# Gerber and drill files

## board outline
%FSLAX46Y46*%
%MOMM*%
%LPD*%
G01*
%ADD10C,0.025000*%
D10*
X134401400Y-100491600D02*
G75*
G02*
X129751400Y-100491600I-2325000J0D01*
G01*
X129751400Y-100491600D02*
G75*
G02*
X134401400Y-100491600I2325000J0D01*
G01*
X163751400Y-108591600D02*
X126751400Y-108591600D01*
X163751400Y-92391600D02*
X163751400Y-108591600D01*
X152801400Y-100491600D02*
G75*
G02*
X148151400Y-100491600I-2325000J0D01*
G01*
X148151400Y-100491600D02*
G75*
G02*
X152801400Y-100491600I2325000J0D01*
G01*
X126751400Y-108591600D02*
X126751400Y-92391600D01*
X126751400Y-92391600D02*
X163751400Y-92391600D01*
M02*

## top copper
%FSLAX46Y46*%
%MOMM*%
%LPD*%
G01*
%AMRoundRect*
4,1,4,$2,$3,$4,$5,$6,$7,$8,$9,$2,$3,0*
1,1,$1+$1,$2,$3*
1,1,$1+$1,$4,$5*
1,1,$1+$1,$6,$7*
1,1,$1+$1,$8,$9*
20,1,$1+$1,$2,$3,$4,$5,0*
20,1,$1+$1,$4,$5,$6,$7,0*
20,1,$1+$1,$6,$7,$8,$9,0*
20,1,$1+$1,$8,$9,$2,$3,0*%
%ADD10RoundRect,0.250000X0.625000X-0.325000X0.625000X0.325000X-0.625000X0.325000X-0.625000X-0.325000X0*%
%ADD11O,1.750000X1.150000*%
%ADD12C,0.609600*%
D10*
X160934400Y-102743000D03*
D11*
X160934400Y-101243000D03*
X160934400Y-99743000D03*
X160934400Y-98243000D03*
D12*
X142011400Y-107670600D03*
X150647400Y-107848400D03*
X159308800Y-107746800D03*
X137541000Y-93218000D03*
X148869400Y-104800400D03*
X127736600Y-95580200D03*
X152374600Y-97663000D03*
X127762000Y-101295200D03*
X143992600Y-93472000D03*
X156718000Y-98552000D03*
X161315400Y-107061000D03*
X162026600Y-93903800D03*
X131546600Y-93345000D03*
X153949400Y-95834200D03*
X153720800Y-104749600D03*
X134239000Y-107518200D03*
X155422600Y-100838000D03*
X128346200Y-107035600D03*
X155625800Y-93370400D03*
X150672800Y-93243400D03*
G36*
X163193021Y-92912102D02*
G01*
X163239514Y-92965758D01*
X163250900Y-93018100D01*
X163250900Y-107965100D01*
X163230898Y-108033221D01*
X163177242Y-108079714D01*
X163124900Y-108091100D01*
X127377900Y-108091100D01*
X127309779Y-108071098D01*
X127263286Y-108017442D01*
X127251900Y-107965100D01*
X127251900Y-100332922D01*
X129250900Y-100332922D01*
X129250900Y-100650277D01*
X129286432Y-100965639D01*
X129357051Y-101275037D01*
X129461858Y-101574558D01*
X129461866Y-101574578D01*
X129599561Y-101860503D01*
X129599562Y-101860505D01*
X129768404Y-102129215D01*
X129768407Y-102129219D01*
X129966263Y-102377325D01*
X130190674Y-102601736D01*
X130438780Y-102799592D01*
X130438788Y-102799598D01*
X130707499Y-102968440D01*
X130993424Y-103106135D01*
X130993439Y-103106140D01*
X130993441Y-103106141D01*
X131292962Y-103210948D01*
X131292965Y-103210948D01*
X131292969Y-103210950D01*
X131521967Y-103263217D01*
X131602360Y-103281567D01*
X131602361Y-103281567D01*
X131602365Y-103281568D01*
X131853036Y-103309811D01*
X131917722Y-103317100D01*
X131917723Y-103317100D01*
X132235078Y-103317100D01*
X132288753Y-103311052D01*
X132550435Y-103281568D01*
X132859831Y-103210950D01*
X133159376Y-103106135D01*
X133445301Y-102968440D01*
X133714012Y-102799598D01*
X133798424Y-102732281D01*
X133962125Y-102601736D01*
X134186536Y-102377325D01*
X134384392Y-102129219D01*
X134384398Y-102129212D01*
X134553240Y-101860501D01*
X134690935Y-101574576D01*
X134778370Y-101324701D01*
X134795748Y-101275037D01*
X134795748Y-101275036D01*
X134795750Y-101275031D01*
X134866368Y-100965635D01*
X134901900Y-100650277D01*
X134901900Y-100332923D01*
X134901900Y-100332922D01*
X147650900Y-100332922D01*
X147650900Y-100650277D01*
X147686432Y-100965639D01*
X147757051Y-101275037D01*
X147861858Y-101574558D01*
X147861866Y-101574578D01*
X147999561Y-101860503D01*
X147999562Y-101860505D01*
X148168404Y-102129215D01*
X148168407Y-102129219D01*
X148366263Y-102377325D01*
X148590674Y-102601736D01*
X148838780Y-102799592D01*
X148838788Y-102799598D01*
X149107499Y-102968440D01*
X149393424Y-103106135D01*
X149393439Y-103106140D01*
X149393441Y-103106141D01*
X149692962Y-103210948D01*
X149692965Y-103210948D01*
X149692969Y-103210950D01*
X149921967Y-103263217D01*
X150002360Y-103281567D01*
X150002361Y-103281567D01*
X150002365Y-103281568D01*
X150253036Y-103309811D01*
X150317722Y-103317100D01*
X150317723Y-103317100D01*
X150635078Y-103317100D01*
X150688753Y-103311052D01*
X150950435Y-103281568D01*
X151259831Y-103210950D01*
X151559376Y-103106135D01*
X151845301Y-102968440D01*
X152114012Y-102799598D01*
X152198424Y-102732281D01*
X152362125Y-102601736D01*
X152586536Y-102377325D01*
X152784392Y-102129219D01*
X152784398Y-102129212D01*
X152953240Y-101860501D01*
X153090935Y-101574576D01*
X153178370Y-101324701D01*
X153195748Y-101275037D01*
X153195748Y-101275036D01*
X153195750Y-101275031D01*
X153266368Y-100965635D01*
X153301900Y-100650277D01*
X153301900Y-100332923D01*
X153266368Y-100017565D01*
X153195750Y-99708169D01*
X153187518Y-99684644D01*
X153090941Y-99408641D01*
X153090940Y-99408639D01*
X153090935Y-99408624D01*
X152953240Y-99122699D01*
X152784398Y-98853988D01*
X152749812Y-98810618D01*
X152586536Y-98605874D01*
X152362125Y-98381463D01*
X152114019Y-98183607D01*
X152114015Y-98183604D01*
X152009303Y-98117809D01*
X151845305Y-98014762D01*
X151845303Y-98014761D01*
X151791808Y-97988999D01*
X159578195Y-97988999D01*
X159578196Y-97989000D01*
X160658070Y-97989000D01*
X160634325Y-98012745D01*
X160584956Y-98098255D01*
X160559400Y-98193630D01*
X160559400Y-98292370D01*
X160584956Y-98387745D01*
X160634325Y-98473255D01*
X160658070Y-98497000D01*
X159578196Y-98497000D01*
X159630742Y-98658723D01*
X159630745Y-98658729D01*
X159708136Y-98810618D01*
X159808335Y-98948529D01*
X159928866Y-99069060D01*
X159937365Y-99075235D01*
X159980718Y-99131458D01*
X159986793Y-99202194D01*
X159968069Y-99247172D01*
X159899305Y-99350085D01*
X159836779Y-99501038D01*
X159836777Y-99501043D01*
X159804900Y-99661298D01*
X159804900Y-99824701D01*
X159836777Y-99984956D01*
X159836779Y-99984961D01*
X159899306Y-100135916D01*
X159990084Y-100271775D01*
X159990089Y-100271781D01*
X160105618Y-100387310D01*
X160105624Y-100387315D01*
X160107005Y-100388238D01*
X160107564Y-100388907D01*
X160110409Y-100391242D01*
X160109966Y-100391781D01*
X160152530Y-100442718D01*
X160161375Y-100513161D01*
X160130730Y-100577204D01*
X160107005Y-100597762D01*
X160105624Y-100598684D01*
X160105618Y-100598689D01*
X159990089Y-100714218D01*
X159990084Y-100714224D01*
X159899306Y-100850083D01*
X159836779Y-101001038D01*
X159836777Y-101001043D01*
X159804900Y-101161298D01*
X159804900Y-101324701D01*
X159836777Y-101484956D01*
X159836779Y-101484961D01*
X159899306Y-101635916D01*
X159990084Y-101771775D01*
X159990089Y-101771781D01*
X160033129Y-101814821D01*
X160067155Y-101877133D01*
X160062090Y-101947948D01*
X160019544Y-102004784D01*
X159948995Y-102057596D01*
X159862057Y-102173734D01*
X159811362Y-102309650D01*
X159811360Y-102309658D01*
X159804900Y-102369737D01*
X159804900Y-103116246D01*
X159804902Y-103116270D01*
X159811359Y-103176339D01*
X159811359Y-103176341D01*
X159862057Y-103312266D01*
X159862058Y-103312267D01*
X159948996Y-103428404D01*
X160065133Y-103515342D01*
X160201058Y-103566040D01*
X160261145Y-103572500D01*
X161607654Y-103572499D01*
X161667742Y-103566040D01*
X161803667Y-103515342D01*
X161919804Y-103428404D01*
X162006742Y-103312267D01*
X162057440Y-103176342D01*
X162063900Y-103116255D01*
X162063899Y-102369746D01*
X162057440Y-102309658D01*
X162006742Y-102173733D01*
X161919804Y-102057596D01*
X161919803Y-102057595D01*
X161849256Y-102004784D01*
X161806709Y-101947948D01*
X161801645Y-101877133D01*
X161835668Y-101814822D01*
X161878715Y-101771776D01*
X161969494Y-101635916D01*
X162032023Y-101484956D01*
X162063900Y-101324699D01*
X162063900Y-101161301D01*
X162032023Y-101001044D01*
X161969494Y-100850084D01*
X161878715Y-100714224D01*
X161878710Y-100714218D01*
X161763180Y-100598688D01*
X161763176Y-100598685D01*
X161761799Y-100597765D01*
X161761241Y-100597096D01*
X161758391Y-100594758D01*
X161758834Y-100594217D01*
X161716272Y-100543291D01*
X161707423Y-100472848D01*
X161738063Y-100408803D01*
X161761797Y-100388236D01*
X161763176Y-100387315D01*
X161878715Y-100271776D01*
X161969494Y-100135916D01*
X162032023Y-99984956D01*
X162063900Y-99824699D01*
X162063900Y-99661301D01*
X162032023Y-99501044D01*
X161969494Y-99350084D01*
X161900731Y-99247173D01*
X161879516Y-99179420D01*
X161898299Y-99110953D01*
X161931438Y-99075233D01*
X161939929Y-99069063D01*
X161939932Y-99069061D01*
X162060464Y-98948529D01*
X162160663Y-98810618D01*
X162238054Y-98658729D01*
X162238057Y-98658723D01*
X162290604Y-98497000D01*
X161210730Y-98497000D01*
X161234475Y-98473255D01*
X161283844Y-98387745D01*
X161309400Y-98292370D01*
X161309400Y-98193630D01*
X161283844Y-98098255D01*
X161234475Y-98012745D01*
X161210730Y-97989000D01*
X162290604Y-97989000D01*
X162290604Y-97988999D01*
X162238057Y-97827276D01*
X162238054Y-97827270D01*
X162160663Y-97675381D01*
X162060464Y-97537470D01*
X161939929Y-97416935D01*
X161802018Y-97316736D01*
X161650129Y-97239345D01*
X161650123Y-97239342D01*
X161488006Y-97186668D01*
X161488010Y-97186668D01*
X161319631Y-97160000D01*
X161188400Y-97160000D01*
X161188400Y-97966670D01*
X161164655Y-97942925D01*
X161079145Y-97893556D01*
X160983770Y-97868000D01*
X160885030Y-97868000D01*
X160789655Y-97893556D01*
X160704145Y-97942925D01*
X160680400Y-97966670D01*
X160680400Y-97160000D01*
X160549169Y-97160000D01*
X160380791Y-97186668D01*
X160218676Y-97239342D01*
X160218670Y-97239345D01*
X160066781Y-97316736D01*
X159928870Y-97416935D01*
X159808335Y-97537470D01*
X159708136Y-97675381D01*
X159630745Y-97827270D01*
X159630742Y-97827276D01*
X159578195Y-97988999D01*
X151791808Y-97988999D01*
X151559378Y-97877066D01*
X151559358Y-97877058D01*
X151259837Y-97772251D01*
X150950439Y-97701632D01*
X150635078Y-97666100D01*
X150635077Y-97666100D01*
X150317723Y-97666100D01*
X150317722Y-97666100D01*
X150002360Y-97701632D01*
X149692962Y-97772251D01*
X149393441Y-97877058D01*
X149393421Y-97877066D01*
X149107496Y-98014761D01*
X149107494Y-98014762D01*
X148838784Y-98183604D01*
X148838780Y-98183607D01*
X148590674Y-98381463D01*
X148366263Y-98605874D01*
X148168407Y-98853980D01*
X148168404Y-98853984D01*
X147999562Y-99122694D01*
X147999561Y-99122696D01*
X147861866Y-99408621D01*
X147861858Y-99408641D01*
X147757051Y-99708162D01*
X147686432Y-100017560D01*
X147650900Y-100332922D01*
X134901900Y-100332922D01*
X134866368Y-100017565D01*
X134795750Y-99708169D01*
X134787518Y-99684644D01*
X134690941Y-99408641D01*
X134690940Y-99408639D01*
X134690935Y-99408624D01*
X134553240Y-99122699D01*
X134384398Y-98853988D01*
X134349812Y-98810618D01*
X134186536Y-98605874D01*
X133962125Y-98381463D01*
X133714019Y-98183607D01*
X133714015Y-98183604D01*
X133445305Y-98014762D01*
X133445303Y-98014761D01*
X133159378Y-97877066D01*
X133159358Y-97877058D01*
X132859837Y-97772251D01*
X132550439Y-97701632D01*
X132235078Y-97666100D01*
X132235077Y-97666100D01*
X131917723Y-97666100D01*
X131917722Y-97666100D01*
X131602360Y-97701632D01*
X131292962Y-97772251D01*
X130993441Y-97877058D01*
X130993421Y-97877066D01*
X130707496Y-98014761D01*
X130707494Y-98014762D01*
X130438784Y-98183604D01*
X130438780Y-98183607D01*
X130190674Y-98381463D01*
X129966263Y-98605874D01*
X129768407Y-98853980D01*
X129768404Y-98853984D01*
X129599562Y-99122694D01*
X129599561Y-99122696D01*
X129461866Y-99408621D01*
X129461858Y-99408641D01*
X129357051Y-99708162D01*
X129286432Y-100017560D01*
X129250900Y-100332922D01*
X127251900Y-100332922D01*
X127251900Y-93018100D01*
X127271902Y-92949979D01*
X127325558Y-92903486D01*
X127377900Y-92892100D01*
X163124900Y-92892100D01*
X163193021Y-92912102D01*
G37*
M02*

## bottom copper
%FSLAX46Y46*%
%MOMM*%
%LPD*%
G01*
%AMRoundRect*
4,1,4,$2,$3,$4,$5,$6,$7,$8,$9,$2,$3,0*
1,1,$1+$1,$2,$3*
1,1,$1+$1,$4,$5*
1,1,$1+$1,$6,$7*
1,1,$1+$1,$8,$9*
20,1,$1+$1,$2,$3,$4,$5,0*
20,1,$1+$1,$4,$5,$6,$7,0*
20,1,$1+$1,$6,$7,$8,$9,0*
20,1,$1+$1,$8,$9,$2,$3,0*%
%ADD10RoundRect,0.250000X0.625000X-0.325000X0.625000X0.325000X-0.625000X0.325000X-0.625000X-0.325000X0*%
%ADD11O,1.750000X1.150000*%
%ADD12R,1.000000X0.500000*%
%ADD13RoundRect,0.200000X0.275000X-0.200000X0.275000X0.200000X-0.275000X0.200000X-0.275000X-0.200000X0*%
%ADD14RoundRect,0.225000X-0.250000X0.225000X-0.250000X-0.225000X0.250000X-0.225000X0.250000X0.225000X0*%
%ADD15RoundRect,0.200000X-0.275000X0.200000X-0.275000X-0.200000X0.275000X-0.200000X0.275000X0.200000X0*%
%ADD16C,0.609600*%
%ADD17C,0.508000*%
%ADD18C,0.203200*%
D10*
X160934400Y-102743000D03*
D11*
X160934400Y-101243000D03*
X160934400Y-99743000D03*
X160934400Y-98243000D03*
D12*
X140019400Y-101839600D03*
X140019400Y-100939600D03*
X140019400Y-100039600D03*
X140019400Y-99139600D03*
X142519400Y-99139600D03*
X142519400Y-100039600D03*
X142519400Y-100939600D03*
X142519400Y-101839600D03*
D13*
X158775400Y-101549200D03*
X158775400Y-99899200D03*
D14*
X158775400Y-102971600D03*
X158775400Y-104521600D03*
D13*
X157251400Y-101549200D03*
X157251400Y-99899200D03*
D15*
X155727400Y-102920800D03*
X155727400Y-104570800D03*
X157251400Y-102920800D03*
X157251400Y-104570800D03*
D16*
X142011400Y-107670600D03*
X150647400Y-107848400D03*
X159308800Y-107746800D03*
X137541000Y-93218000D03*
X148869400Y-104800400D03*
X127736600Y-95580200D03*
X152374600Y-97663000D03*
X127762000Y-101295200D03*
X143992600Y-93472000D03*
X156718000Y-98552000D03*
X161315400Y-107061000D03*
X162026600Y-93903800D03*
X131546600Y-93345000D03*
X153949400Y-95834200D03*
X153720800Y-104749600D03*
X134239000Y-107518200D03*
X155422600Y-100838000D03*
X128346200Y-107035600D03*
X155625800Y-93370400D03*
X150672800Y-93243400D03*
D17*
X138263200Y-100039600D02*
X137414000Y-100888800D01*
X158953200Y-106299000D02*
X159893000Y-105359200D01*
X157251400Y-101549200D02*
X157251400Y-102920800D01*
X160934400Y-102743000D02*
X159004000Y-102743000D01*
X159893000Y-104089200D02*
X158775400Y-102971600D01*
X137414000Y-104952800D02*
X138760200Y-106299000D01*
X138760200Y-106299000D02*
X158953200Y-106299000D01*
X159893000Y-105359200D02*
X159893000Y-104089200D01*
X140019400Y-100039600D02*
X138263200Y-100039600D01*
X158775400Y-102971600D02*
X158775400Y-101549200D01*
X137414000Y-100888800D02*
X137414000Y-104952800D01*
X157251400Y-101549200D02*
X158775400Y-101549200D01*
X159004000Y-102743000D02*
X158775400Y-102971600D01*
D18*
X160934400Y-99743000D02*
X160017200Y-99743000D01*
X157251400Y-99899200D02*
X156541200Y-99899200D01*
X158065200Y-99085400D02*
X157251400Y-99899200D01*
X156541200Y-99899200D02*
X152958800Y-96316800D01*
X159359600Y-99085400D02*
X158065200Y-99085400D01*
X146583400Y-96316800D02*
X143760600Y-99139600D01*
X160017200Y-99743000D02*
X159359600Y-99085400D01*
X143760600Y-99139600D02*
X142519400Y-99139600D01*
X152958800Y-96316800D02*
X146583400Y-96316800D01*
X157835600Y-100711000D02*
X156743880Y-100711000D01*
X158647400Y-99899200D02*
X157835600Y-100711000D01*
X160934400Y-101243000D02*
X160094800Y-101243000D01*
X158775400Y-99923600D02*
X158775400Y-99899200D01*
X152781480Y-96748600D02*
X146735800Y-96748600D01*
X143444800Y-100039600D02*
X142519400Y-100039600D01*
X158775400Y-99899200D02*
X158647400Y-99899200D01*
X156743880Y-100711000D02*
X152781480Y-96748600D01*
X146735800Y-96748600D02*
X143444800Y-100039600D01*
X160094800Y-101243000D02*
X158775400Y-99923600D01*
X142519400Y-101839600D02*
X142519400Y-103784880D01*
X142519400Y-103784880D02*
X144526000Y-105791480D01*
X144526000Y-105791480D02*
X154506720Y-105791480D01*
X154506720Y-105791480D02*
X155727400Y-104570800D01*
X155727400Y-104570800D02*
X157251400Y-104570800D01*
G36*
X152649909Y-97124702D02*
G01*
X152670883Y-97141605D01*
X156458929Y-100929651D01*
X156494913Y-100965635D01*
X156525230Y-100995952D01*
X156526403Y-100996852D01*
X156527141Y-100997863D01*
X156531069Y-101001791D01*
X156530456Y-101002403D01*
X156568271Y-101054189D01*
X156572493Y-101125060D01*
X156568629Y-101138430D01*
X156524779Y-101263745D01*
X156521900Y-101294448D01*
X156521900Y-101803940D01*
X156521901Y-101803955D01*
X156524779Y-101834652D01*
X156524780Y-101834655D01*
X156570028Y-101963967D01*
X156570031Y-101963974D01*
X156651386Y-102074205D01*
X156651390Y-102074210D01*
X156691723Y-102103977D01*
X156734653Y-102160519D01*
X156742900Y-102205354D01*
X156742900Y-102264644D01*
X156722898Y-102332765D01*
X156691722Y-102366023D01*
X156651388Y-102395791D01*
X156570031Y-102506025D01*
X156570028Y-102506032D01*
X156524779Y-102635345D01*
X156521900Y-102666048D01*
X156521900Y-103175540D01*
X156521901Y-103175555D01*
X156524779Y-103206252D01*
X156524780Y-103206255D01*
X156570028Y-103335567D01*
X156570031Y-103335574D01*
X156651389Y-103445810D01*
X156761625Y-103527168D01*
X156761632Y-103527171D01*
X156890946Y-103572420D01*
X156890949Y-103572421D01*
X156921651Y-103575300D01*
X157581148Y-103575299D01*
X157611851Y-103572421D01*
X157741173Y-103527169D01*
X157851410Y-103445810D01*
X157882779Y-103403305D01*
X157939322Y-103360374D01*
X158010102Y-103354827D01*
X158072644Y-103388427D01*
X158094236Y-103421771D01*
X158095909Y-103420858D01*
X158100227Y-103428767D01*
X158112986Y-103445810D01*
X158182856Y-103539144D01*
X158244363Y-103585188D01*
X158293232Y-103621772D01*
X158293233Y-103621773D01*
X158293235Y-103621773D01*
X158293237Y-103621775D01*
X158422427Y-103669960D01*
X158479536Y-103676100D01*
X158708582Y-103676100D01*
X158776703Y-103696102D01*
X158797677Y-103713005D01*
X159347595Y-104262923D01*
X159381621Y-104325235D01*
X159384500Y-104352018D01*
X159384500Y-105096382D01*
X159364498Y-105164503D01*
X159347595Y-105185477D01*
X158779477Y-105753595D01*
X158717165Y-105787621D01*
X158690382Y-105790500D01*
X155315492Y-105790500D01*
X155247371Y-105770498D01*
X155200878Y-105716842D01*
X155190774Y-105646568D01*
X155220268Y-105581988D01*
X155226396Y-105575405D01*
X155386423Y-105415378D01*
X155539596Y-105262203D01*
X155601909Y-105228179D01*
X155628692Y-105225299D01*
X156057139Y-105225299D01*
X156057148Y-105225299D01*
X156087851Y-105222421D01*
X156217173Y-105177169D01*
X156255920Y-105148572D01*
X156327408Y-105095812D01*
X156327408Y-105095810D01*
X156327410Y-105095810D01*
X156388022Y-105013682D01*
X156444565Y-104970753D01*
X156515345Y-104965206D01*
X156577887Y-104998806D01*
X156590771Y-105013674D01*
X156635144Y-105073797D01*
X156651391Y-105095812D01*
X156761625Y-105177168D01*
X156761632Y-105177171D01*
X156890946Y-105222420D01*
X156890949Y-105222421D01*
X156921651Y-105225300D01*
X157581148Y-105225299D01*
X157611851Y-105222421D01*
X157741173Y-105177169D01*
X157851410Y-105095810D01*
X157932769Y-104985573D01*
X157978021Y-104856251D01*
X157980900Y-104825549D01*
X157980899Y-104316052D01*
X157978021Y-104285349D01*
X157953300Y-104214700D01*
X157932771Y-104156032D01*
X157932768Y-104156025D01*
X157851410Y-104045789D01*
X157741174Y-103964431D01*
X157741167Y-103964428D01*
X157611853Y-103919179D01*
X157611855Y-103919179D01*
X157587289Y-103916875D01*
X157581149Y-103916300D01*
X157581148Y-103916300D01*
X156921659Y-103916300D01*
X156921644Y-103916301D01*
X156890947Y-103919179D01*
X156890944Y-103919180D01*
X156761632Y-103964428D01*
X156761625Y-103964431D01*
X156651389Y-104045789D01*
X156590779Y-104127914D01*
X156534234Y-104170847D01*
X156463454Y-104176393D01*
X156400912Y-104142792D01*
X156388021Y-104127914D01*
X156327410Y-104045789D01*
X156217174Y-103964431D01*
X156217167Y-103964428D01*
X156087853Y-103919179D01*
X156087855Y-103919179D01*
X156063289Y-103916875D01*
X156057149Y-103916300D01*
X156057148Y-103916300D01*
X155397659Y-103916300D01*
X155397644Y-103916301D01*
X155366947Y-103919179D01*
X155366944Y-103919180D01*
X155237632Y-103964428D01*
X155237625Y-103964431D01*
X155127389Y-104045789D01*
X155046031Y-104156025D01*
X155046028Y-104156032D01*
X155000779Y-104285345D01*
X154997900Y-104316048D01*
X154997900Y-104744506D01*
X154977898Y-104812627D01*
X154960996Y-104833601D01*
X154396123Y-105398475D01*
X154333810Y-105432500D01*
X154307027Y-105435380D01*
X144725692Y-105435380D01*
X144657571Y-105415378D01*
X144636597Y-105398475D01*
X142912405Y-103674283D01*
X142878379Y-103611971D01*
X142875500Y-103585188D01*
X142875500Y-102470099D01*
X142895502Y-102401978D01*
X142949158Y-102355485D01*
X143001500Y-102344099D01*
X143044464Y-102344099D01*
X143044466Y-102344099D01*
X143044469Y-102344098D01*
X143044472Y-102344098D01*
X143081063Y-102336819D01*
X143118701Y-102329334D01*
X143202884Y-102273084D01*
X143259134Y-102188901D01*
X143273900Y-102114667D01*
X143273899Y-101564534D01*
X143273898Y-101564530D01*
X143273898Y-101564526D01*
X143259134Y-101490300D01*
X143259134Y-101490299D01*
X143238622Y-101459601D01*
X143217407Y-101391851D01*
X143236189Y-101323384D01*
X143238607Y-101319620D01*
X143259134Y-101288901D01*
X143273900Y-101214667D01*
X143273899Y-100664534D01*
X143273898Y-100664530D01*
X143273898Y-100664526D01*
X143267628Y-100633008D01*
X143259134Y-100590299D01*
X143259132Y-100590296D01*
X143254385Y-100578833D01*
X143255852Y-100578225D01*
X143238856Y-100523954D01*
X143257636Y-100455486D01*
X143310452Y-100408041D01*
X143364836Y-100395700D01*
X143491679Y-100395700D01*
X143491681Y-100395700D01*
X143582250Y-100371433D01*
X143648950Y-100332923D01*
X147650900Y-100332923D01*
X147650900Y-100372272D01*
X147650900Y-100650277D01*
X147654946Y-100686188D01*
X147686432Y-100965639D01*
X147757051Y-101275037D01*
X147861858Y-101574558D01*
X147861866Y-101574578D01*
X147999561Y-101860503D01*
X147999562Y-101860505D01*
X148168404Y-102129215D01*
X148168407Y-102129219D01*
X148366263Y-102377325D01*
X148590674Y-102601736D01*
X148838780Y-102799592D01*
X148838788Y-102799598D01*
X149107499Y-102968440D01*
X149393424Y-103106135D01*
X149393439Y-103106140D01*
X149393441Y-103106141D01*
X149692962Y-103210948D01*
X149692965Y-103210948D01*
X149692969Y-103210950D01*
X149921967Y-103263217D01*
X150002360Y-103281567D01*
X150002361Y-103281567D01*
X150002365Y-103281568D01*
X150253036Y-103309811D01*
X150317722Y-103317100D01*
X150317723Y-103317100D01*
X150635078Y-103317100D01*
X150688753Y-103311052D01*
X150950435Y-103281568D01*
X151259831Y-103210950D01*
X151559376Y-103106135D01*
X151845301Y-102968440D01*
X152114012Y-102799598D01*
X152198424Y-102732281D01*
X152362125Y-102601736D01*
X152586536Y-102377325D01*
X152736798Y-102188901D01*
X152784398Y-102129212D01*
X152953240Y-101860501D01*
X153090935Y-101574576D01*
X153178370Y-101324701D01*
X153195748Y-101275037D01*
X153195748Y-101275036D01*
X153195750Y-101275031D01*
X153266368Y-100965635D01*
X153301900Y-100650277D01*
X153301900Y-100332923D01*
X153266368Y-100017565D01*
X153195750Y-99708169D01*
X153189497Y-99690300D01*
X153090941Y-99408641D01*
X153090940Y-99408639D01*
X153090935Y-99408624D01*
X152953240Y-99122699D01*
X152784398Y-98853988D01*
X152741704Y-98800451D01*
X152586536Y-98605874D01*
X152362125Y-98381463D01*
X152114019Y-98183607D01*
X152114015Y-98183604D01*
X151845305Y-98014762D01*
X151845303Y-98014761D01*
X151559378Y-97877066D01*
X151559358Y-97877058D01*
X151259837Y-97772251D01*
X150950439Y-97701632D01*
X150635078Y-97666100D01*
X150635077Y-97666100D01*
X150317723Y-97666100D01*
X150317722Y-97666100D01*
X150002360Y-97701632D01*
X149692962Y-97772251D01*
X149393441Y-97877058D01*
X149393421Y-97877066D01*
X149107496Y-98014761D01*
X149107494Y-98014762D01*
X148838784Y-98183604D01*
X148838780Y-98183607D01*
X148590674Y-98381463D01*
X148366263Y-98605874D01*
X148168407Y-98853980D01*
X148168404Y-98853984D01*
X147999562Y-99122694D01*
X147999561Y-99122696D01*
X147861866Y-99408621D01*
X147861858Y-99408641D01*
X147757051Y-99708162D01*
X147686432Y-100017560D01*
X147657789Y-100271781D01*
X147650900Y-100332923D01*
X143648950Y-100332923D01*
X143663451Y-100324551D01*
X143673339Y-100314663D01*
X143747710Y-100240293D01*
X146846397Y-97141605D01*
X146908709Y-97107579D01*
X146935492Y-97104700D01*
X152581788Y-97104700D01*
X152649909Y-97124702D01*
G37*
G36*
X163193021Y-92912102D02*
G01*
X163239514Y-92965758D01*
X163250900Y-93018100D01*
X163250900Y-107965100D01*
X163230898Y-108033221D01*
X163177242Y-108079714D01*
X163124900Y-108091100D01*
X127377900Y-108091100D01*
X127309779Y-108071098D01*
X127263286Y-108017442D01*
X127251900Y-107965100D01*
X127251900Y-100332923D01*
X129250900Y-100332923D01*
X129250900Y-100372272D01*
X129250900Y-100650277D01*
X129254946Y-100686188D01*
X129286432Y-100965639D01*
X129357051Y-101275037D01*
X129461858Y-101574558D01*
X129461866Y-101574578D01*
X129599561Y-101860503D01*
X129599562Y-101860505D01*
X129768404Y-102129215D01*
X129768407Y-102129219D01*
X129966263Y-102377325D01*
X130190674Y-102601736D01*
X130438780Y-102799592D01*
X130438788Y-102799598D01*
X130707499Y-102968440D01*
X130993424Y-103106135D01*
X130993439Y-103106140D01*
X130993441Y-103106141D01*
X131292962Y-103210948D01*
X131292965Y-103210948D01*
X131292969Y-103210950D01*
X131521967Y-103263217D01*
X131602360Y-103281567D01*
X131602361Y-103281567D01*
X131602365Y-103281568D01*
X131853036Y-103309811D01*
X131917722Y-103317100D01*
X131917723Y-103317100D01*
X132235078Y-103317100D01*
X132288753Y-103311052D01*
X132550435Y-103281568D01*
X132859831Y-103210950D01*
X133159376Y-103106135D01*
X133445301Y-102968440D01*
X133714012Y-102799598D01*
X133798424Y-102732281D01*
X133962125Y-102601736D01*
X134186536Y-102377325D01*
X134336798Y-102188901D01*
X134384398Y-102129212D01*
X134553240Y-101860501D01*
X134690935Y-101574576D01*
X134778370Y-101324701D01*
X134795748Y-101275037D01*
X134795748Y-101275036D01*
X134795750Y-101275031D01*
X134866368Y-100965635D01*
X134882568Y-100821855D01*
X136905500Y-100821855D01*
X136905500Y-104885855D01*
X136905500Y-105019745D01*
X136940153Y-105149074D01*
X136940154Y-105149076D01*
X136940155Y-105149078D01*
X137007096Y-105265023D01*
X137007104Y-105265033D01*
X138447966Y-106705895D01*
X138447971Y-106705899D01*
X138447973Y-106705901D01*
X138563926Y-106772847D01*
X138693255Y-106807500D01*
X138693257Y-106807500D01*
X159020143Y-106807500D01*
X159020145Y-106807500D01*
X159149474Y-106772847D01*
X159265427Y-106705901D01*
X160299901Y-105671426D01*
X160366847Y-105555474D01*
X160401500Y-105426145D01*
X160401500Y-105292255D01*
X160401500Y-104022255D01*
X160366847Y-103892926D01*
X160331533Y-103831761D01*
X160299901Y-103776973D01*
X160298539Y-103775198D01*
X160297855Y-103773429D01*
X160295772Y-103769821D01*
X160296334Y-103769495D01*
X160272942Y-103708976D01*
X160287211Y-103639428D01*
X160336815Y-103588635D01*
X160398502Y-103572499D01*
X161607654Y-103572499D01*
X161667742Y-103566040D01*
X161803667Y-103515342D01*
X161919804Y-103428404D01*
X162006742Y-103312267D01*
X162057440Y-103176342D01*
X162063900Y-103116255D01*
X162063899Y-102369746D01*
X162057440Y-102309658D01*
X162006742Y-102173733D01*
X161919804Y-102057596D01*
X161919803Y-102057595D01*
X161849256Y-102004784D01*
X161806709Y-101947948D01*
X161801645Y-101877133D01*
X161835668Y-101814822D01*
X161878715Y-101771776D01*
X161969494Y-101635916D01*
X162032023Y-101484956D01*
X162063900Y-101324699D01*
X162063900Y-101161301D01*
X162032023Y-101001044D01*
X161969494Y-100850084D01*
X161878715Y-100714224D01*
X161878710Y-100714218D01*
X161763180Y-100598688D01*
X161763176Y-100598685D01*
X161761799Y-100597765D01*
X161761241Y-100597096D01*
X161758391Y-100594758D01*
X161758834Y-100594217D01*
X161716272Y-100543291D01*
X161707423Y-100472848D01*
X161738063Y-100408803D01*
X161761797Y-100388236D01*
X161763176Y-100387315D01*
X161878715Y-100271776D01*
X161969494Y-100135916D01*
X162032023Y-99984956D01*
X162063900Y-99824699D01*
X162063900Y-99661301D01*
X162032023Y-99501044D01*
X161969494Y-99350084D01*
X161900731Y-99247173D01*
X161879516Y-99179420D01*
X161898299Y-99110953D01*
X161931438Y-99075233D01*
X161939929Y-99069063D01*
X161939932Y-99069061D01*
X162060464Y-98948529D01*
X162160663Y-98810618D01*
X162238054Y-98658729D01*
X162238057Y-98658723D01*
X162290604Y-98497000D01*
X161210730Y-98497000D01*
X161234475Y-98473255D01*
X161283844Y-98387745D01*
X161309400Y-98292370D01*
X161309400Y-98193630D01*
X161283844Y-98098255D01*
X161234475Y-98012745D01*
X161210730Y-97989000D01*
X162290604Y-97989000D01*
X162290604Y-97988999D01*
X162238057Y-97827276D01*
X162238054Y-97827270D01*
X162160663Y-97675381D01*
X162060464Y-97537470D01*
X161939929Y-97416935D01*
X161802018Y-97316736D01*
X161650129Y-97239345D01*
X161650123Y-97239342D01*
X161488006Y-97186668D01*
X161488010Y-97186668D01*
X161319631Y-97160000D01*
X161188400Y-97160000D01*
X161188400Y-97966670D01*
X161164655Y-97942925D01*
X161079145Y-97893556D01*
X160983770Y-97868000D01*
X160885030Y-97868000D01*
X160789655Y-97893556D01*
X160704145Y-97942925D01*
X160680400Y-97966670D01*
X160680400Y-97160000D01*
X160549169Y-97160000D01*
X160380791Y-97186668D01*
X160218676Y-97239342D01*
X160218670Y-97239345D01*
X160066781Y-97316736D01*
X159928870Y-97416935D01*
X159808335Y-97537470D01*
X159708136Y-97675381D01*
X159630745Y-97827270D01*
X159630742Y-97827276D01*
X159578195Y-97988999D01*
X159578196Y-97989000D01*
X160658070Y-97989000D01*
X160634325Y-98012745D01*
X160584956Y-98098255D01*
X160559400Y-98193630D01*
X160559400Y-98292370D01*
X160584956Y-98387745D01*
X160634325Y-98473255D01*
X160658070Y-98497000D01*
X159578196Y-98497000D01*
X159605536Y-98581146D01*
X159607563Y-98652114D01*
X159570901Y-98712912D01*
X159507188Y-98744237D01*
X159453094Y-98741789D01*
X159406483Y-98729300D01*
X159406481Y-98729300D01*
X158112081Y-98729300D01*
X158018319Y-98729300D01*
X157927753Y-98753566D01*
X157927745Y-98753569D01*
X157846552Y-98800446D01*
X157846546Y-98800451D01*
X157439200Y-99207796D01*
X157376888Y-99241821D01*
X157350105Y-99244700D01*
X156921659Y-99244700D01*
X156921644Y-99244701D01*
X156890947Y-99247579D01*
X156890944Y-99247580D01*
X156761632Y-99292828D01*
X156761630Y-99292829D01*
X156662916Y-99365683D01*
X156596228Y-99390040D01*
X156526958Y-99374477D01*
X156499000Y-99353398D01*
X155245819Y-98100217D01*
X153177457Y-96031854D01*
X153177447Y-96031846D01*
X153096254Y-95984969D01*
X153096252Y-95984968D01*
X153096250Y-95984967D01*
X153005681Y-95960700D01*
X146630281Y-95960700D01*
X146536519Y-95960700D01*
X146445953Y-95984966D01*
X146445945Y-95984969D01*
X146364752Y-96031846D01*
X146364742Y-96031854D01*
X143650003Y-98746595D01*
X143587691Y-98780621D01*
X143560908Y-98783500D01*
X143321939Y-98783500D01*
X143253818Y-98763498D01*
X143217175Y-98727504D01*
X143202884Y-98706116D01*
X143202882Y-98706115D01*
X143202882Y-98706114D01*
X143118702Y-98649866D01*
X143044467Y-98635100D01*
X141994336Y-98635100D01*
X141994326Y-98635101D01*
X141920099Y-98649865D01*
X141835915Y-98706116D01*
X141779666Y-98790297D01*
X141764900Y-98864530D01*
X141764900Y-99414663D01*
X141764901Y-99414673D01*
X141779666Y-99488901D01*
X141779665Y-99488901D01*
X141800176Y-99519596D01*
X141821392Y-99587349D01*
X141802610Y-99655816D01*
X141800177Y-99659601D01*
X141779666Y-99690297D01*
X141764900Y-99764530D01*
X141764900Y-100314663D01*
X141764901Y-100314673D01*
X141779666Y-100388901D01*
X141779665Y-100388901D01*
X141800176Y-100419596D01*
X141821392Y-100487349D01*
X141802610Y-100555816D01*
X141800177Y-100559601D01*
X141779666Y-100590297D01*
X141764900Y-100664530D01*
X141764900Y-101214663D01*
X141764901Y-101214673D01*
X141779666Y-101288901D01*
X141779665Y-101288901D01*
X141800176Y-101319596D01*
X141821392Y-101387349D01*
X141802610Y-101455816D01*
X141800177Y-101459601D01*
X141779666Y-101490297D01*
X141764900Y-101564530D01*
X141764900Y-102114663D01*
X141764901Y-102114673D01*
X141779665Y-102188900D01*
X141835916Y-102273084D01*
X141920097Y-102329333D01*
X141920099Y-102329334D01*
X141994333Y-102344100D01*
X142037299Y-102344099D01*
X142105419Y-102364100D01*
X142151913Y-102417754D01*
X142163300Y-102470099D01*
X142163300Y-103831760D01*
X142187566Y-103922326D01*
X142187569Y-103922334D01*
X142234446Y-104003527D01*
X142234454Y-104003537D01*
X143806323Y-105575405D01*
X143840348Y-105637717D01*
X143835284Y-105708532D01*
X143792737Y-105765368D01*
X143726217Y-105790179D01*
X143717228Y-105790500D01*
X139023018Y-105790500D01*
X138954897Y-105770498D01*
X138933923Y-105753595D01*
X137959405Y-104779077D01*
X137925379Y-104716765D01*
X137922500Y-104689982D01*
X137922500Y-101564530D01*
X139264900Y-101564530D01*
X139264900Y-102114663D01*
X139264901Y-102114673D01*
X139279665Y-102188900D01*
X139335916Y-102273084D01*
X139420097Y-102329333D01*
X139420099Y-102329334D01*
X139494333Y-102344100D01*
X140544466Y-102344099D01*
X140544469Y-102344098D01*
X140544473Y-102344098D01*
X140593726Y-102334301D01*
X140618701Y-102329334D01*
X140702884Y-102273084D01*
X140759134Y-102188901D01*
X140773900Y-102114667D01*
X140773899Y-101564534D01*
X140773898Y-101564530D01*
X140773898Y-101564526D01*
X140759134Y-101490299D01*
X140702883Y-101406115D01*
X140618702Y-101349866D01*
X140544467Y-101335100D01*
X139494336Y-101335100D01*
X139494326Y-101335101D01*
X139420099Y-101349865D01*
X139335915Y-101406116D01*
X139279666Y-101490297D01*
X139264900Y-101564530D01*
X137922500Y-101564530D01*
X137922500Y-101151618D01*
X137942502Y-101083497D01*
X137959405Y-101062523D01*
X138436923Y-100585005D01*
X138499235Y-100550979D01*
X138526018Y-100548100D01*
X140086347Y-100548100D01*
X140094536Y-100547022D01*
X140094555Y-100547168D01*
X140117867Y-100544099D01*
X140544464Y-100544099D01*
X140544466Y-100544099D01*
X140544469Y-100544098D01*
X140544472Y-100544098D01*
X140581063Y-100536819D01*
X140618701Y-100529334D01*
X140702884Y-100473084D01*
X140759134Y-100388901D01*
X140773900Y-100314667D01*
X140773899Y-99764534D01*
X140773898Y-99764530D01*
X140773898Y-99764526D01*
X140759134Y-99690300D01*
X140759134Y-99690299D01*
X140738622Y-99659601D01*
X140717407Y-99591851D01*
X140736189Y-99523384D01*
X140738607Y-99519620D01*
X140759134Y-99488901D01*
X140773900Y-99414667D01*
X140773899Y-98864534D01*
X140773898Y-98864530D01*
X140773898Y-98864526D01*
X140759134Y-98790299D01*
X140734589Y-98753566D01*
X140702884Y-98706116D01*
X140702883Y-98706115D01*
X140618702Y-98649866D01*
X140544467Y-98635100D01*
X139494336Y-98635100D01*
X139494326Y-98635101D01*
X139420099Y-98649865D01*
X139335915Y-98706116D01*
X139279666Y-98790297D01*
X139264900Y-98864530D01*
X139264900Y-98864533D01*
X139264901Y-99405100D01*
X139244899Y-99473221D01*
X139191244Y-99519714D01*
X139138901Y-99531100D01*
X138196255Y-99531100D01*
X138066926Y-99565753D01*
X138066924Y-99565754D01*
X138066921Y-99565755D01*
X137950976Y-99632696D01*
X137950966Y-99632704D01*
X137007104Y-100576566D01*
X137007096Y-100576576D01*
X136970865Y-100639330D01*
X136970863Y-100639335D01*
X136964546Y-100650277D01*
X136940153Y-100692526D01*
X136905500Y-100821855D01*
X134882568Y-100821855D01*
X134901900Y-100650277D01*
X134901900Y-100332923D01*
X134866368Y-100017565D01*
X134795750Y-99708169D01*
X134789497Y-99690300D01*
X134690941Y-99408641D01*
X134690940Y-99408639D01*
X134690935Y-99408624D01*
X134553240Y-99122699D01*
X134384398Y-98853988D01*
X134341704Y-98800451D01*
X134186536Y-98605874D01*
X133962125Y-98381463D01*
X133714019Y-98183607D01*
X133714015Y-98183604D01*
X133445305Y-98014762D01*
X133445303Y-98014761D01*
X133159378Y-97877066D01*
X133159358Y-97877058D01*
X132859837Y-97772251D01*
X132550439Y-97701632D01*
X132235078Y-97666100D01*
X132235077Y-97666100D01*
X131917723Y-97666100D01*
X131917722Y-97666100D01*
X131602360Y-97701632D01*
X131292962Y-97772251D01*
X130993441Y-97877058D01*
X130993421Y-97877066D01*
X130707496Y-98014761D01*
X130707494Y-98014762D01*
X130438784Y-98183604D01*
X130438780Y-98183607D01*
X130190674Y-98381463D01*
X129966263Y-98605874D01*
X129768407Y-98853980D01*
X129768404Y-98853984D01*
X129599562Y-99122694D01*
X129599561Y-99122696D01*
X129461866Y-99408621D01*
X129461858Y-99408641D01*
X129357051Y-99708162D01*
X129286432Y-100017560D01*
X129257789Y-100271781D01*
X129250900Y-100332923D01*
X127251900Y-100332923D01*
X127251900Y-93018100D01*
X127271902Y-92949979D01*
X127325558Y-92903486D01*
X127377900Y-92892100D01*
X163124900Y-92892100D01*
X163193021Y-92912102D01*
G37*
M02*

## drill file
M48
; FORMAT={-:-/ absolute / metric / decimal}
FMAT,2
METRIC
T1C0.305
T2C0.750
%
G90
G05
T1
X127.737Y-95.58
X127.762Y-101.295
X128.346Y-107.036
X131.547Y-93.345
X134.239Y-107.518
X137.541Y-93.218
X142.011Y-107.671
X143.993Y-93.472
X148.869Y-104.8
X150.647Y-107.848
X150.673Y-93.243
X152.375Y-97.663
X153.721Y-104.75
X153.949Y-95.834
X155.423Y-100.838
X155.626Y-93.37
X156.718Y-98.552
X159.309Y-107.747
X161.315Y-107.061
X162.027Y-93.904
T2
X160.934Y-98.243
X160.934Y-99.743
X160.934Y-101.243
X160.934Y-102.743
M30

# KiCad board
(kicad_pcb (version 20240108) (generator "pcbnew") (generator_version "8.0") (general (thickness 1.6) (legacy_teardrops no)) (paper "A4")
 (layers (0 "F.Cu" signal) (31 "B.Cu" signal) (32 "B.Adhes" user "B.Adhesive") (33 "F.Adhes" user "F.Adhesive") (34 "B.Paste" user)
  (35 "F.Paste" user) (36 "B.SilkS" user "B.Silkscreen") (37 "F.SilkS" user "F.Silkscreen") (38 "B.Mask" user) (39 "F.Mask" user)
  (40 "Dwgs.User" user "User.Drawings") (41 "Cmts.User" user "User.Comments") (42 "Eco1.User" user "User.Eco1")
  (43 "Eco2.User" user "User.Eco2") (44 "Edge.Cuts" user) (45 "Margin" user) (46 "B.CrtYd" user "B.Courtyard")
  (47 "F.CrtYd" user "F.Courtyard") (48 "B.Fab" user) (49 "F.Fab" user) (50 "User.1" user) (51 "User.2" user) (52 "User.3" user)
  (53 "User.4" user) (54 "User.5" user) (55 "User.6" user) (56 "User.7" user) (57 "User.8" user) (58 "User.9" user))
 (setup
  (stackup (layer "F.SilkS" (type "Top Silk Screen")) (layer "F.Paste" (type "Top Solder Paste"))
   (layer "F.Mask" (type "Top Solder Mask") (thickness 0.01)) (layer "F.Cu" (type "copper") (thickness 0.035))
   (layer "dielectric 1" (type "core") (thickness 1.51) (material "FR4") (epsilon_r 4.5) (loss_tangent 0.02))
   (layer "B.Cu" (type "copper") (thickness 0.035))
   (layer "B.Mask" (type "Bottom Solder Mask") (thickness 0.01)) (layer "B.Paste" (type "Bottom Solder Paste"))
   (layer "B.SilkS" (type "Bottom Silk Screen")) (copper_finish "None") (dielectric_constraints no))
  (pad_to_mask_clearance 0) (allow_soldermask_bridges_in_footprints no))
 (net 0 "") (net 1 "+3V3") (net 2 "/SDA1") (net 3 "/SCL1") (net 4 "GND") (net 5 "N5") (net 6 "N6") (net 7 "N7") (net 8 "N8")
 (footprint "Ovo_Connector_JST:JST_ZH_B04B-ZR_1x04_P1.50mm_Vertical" (layer "F.Cu") (at 160.9344 102.743 90)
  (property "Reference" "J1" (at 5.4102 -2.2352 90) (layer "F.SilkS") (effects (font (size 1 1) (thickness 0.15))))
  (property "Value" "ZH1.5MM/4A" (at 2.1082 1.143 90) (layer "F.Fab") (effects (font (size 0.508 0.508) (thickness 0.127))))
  (pad "1" thru_hole roundrect (at 0 0 90) (size 1.15 1.75) (drill 0.75) (layers "*.Cu" "*.Mask") (remove_unused_layers no)
   (roundrect_rratio 0.2173913043) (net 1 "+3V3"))
  (pad "2" thru_hole oval (at 1.5 0 90) (size 1.15 1.75) (drill 0.75) (layers "*.Cu" "*.Mask") (remove_unused_layers no) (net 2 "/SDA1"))
  (pad "3" thru_hole oval (at 3 0 90) (size 1.15 1.75) (drill 0.75) (layers "*.Cu" "*.Mask") (remove_unused_layers no) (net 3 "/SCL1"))
  (pad "4" thru_hole oval (at 4.5 0 90) (size 1.15 1.75) (drill 0.75) (layers "*.Cu" "*.Mask") (remove_unused_layers no) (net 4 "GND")))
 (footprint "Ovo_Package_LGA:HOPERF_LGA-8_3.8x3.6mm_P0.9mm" (layer "B.Cu") (at 141.2694 100.4896)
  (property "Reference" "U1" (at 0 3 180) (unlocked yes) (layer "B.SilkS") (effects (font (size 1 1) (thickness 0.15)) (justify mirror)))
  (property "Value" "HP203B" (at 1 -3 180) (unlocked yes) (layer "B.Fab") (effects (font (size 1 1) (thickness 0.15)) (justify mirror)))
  (pad "1" smd rect (at -1.25 1.35) (size 1 0.5) (layers "B.Cu" "B.Paste" "B.Mask") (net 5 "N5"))
  (pad "2" smd rect (at -1.25 0.45) (size 1 0.5) (layers "B.Cu" "B.Paste" "B.Mask") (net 4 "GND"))
  (pad "3" smd rect (at -1.25 -0.45) (size 1 0.5) (layers "B.Cu" "B.Paste" "B.Mask") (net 1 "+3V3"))
  (pad "4" smd rect (at -1.25 -1.35) (size 1 0.5) (layers "B.Cu" "B.Paste" "B.Mask") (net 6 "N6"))
  (pad "5" smd rect (at 1.25 -1.35) (size 1 0.5) (layers "B.Cu" "B.Paste" "B.Mask") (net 3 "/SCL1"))
  (pad "6" smd rect (at 1.25 -0.45) (size 1 0.5) (layers "B.Cu" "B.Paste" "B.Mask") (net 2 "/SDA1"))
  (pad "7" smd rect (at 1.25 0.45) (size 1 0.5) (layers "B.Cu" "B.Paste" "B.Mask") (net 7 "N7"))
  (pad "8" smd rect (at 1.25 1.35) (size 1 0.5) (layers "B.Cu" "B.Paste" "B.Mask") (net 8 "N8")))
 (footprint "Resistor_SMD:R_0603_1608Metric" (layer "B.Cu") (at 158.7754 100.7242 90)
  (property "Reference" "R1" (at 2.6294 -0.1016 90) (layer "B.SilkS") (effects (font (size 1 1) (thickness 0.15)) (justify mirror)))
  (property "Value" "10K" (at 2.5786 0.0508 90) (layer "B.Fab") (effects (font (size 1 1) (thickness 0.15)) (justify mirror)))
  (pad "1" smd roundrect (at -0.825 0 90) (size 0.8 0.95) (layers "B.Cu" "B.Paste" "B.Mask") (roundrect_rratio 0.25) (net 1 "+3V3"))
  (pad "2" smd roundrect (at 0.825 0 90) (size 0.8 0.95) (layers "B.Cu" "B.Paste" "B.Mask") (roundrect_rratio 0.25) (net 2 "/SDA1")))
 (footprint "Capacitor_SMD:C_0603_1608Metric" (layer "B.Cu") (at 158.7754 103.7466 -90)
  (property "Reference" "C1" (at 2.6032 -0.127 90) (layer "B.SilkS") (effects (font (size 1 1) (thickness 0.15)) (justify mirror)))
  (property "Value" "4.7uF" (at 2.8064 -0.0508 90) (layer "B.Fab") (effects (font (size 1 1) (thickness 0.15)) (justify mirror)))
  (pad "1" smd roundrect (at -0.775 0 270) (size 0.9 0.95) (layers "B.Cu" "B.Paste" "B.Mask") (roundrect_rratio 0.25) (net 1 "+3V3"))
  (pad "2" smd roundrect (at 0.775 0 270) (size 0.9 0.95) (layers "B.Cu" "B.Paste" "B.Mask") (roundrect_rratio 0.25) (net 4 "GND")))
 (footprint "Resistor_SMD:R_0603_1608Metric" (layer "B.Cu") (at 157.2514 100.7242 90)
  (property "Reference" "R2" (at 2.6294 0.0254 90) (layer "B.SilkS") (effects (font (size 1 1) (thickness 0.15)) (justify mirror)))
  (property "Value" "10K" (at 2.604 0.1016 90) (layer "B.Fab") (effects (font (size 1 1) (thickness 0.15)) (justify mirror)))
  (pad "1" smd roundrect (at -0.825 0 90) (size 0.8 0.95) (layers "B.Cu" "B.Paste" "B.Mask") (roundrect_rratio 0.25) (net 1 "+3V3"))
  (pad "2" smd roundrect (at 0.825 0 90) (size 0.8 0.95) (layers "B.Cu" "B.Paste" "B.Mask") (roundrect_rratio 0.25) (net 3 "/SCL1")))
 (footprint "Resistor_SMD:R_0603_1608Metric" (layer "B.Cu") (at 155.7274 103.7458 -90)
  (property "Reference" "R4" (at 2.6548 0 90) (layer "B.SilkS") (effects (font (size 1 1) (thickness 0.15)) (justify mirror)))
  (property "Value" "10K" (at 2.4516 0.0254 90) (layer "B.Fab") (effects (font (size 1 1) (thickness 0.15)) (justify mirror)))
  (pad "1" smd roundrect (at -0.825 0 270) (size 0.8 0.95) (layers "B.Cu" "B.Paste" "B.Mask") (roundrect_rratio 0.25) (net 4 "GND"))
  (pad "2" smd roundrect (at 0.825 0 270) (size 0.8 0.95) (layers "B.Cu" "B.Paste" "B.Mask") (roundrect_rratio 0.25) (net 8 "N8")))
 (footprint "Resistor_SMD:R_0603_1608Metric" (layer "B.Cu") (at 157.2514 103.7458 -90)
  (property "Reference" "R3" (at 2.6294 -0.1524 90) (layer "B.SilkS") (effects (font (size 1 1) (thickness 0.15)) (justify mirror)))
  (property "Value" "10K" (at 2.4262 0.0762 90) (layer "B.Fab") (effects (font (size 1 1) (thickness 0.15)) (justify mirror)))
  (pad "1" smd roundrect (at -0.825 0 270) (size 0.8 0.95) (layers "B.Cu" "B.Paste" "B.Mask") (roundrect_rratio 0.25) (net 1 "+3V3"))
  (pad "2" smd roundrect (at 0.825 0 270) (size 0.8 0.95) (layers "B.Cu" "B.Paste" "B.Mask") (roundrect_rratio 0.25) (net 8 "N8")))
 (gr_circle (center 132.0764 100.4916) (end 134.4014 100.4916) (stroke (width 0.025) (type solid)) (fill none) (layer "Edge.Cuts"))
 (gr_line (start 163.7514 108.5916) (end 126.7514 108.5916) (stroke (width 0.025) (type solid)) (layer "Edge.Cuts"))
 (gr_line (start 163.7514 92.3916) (end 163.7514 108.5916) (stroke (width 0.025) (type solid)) (layer "Edge.Cuts"))
 (gr_circle (center 150.4764 100.4916) (end 152.8014 100.4916) (stroke (width 0.025) (type solid)) (fill none) (layer "Edge.Cuts"))
 (gr_line (start 126.7514 108.5916) (end 126.7514 92.3916) (stroke (width 0.025) (type solid)) (layer "Edge.Cuts"))
 (gr_line (start 126.7514 92.3916) (end 163.7514 92.3916) (stroke (width 0.025) (type solid)) (layer "Edge.Cuts"))
 (segment (start 138.2632 100.0396) (end 137.414 100.8888) (width 0.508) (layer "B.Cu") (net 1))
 (segment (start 158.9532 106.299) (end 159.893 105.3592) (width 0.508) (layer "B.Cu") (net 1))
 (segment (start 157.2514 101.5492) (end 157.2514 102.9208) (width 0.508) (layer "B.Cu") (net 1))
 (segment (start 160.9344 102.743) (end 159.004 102.743) (width 0.508) (layer "B.Cu") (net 1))
 (segment (start 159.893 104.0892) (end 158.7754 102.9716) (width 0.508) (layer "B.Cu") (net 1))
 (segment (start 137.414 104.9528) (end 138.7602 106.299) (width 0.508) (layer "B.Cu") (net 1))
 (segment (start 138.7602 106.299) (end 158.9532 106.299) (width 0.508) (layer "B.Cu") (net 1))
 (segment (start 159.893 105.3592) (end 159.893 104.0892) (width 0.508) (layer "B.Cu") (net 1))
 (segment (start 140.0194 100.0396) (end 138.2632 100.0396) (width 0.508) (layer "B.Cu") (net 1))
 (segment (start 158.7754 102.9716) (end 158.7754 101.5492) (width 0.508) (layer "B.Cu") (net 1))
 (segment (start 137.414 100.8888) (end 137.414 104.9528) (width 0.508) (layer "B.Cu") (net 1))
 (segment (start 157.2514 101.5492) (end 158.7754 101.5492) (width 0.508) (layer "B.Cu") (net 1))
 (segment (start 159.004 102.743) (end 158.7754 102.9716) (width 0.508) (layer "B.Cu") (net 1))
 (via (at 142.0114 107.6706) (size 0.6096) (drill 0.3048) (layers "F.Cu" "B.Cu") (free yes) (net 4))
 (via (at 150.6474 107.8484) (size 0.6096) (drill 0.3048) (layers "F.Cu" "B.Cu") (free yes) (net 4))
 (via (at 159.3088 107.7468) (size 0.6096) (drill 0.3048) (layers "F.Cu" "B.Cu") (free yes) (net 4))
 (via (at 137.541 93.218) (size 0.6096) (drill 0.3048) (layers "F.Cu" "B.Cu") (free yes) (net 4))
 (via (at 148.8694 104.8004) (size 0.6096) (drill 0.3048) (layers "F.Cu" "B.Cu") (free yes) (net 4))
 (via (at 127.7366 95.5802) (size 0.6096) (drill 0.3048) (layers "F.Cu" "B.Cu") (free yes) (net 4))
 (via (at 152.3746 97.663) (size 0.6096) (drill 0.3048) (layers "F.Cu" "B.Cu") (free yes) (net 4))
 (via (at 127.762 101.2952) (size 0.6096) (drill 0.3048) (layers "F.Cu" "B.Cu") (free yes) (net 4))
 (via (at 143.9926 93.472) (size 0.6096) (drill 0.3048) (layers "F.Cu" "B.Cu") (free yes) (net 4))
 (via (at 156.718 98.552) (size 0.6096) (drill 0.3048) (layers "F.Cu" "B.Cu") (free yes) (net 4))
 (via (at 161.3154 107.061) (size 0.6096) (drill 0.3048) (layers "F.Cu" "B.Cu") (free yes) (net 4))
 (via (at 162.0266 93.9038) (size 0.6096) (drill 0.3048) (layers "F.Cu" "B.Cu") (free yes) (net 4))
 (via (at 131.5466 93.345) (size 0.6096) (drill 0.3048) (layers "F.Cu" "B.Cu") (free yes) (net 4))
 (via (at 153.9494 95.8342) (size 0.6096) (drill 0.3048) (layers "F.Cu" "B.Cu") (free yes) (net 4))
 (via (at 153.7208 104.7496) (size 0.6096) (drill 0.3048) (layers "F.Cu" "B.Cu") (free yes) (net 4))
 (via (at 134.239 107.5182) (size 0.6096) (drill 0.3048) (layers "F.Cu" "B.Cu") (free yes) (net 4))
 (via (at 155.4226 100.838) (size 0.6096) (drill 0.3048) (layers "F.Cu" "B.Cu") (free yes) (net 4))
 (via (at 128.3462 107.0356) (size 0.6096) (drill 0.3048) (layers "F.Cu" "B.Cu") (free yes) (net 4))
 (via (at 155.6258 93.3704) (size 0.6096) (drill 0.3048) (layers "F.Cu" "B.Cu") (free yes) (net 4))
 (via (at 150.6728 93.2434) (size 0.6096) (drill 0.3048) (layers "F.Cu" "B.Cu") (free yes) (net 4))
 (segment (start 160.9344 99.743) (end 160.0172 99.743) (width 0.2032) (layer "B.Cu") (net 3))
 (segment (start 157.2514 99.8992) (end 156.5412 99.8992) (width 0.2032) (layer "B.Cu") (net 3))
 (segment (start 158.0652 99.0854) (end 157.2514 99.8992) (width 0.2032) (layer "B.Cu") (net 3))
 (segment (start 156.5412 99.8992) (end 152.9588 96.3168) (width 0.2032) (layer "B.Cu") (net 3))
 (segment (start 159.3596 99.0854) (end 158.0652 99.0854) (width 0.2032) (layer "B.Cu") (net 3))
 (segment (start 146.5834 96.3168) (end 143.7606 99.1396) (width 0.2032) (layer "B.Cu") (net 3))
 (segment (start 160.0172 99.743) (end 159.3596 99.0854) (width 0.2032) (layer "B.Cu") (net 3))
 (segment (start 143.7606 99.1396) (end 142.5194 99.1396) (width 0.2032) (layer "B.Cu") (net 3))
 (segment (start 152.9588 96.3168) (end 146.5834 96.3168) (width 0.2032) (layer "B.Cu") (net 3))
 (segment (start 157.8356 100.711) (end 156.74388 100.711) (width 0.2032) (layer "B.Cu") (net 2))
 (segment (start 158.6474 99.8992) (end 157.8356 100.711) (width 0.2032) (layer "B.Cu") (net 2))
 (segment (start 160.9344 101.243) (end 160.0948 101.243) (width 0.2032) (layer "B.Cu") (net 2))
 (segment (start 158.7754 99.9236) (end 158.7754 99.8992) (width 0.2032) (layer "B.Cu") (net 2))
 (segment (start 152.78148 96.7486) (end 146.7358 96.7486) (width 0.2032) (layer "B.Cu") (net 2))
 (segment (start 143.4448 100.0396) (end 142.5194 100.0396) (width 0.2032) (layer "B.Cu") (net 2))
 (segment (start 158.7754 99.8992) (end 158.6474 99.8992) (width 0.2032) (layer "B.Cu") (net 2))
 (segment (start 156.74388 100.711) (end 152.78148 96.7486) (width 0.2032) (layer "B.Cu") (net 2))
 (segment (start 146.7358 96.7486) (end 143.4448 100.0396) (width 0.2032) (layer "B.Cu") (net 2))
 (segment (start 160.0948 101.243) (end 158.7754 99.9236) (width 0.2032) (layer "B.Cu") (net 2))
 (segment (start 142.5194 101.8396) (end 142.5194 103.78488) (width 0.2032) (layer "B.Cu") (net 8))
 (segment (start 142.5194 103.78488) (end 144.526 105.79148) (width 0.2032) (layer "B.Cu") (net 8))
 (segment (start 144.526 105.79148) (end 154.50672 105.79148) (width 0.2032) (layer "B.Cu") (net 8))
 (segment (start 154.50672 105.79148) (end 155.7274 104.5708) (width 0.2032) (layer "B.Cu") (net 8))
 (segment (start 155.7274 104.5708) (end 157.2514 104.5708) (width 0.2032) (layer "B.Cu") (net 8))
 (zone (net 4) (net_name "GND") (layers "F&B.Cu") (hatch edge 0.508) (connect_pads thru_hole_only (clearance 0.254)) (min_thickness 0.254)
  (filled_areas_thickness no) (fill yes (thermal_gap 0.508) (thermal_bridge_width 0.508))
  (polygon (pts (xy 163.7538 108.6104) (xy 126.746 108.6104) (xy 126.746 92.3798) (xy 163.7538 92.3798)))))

